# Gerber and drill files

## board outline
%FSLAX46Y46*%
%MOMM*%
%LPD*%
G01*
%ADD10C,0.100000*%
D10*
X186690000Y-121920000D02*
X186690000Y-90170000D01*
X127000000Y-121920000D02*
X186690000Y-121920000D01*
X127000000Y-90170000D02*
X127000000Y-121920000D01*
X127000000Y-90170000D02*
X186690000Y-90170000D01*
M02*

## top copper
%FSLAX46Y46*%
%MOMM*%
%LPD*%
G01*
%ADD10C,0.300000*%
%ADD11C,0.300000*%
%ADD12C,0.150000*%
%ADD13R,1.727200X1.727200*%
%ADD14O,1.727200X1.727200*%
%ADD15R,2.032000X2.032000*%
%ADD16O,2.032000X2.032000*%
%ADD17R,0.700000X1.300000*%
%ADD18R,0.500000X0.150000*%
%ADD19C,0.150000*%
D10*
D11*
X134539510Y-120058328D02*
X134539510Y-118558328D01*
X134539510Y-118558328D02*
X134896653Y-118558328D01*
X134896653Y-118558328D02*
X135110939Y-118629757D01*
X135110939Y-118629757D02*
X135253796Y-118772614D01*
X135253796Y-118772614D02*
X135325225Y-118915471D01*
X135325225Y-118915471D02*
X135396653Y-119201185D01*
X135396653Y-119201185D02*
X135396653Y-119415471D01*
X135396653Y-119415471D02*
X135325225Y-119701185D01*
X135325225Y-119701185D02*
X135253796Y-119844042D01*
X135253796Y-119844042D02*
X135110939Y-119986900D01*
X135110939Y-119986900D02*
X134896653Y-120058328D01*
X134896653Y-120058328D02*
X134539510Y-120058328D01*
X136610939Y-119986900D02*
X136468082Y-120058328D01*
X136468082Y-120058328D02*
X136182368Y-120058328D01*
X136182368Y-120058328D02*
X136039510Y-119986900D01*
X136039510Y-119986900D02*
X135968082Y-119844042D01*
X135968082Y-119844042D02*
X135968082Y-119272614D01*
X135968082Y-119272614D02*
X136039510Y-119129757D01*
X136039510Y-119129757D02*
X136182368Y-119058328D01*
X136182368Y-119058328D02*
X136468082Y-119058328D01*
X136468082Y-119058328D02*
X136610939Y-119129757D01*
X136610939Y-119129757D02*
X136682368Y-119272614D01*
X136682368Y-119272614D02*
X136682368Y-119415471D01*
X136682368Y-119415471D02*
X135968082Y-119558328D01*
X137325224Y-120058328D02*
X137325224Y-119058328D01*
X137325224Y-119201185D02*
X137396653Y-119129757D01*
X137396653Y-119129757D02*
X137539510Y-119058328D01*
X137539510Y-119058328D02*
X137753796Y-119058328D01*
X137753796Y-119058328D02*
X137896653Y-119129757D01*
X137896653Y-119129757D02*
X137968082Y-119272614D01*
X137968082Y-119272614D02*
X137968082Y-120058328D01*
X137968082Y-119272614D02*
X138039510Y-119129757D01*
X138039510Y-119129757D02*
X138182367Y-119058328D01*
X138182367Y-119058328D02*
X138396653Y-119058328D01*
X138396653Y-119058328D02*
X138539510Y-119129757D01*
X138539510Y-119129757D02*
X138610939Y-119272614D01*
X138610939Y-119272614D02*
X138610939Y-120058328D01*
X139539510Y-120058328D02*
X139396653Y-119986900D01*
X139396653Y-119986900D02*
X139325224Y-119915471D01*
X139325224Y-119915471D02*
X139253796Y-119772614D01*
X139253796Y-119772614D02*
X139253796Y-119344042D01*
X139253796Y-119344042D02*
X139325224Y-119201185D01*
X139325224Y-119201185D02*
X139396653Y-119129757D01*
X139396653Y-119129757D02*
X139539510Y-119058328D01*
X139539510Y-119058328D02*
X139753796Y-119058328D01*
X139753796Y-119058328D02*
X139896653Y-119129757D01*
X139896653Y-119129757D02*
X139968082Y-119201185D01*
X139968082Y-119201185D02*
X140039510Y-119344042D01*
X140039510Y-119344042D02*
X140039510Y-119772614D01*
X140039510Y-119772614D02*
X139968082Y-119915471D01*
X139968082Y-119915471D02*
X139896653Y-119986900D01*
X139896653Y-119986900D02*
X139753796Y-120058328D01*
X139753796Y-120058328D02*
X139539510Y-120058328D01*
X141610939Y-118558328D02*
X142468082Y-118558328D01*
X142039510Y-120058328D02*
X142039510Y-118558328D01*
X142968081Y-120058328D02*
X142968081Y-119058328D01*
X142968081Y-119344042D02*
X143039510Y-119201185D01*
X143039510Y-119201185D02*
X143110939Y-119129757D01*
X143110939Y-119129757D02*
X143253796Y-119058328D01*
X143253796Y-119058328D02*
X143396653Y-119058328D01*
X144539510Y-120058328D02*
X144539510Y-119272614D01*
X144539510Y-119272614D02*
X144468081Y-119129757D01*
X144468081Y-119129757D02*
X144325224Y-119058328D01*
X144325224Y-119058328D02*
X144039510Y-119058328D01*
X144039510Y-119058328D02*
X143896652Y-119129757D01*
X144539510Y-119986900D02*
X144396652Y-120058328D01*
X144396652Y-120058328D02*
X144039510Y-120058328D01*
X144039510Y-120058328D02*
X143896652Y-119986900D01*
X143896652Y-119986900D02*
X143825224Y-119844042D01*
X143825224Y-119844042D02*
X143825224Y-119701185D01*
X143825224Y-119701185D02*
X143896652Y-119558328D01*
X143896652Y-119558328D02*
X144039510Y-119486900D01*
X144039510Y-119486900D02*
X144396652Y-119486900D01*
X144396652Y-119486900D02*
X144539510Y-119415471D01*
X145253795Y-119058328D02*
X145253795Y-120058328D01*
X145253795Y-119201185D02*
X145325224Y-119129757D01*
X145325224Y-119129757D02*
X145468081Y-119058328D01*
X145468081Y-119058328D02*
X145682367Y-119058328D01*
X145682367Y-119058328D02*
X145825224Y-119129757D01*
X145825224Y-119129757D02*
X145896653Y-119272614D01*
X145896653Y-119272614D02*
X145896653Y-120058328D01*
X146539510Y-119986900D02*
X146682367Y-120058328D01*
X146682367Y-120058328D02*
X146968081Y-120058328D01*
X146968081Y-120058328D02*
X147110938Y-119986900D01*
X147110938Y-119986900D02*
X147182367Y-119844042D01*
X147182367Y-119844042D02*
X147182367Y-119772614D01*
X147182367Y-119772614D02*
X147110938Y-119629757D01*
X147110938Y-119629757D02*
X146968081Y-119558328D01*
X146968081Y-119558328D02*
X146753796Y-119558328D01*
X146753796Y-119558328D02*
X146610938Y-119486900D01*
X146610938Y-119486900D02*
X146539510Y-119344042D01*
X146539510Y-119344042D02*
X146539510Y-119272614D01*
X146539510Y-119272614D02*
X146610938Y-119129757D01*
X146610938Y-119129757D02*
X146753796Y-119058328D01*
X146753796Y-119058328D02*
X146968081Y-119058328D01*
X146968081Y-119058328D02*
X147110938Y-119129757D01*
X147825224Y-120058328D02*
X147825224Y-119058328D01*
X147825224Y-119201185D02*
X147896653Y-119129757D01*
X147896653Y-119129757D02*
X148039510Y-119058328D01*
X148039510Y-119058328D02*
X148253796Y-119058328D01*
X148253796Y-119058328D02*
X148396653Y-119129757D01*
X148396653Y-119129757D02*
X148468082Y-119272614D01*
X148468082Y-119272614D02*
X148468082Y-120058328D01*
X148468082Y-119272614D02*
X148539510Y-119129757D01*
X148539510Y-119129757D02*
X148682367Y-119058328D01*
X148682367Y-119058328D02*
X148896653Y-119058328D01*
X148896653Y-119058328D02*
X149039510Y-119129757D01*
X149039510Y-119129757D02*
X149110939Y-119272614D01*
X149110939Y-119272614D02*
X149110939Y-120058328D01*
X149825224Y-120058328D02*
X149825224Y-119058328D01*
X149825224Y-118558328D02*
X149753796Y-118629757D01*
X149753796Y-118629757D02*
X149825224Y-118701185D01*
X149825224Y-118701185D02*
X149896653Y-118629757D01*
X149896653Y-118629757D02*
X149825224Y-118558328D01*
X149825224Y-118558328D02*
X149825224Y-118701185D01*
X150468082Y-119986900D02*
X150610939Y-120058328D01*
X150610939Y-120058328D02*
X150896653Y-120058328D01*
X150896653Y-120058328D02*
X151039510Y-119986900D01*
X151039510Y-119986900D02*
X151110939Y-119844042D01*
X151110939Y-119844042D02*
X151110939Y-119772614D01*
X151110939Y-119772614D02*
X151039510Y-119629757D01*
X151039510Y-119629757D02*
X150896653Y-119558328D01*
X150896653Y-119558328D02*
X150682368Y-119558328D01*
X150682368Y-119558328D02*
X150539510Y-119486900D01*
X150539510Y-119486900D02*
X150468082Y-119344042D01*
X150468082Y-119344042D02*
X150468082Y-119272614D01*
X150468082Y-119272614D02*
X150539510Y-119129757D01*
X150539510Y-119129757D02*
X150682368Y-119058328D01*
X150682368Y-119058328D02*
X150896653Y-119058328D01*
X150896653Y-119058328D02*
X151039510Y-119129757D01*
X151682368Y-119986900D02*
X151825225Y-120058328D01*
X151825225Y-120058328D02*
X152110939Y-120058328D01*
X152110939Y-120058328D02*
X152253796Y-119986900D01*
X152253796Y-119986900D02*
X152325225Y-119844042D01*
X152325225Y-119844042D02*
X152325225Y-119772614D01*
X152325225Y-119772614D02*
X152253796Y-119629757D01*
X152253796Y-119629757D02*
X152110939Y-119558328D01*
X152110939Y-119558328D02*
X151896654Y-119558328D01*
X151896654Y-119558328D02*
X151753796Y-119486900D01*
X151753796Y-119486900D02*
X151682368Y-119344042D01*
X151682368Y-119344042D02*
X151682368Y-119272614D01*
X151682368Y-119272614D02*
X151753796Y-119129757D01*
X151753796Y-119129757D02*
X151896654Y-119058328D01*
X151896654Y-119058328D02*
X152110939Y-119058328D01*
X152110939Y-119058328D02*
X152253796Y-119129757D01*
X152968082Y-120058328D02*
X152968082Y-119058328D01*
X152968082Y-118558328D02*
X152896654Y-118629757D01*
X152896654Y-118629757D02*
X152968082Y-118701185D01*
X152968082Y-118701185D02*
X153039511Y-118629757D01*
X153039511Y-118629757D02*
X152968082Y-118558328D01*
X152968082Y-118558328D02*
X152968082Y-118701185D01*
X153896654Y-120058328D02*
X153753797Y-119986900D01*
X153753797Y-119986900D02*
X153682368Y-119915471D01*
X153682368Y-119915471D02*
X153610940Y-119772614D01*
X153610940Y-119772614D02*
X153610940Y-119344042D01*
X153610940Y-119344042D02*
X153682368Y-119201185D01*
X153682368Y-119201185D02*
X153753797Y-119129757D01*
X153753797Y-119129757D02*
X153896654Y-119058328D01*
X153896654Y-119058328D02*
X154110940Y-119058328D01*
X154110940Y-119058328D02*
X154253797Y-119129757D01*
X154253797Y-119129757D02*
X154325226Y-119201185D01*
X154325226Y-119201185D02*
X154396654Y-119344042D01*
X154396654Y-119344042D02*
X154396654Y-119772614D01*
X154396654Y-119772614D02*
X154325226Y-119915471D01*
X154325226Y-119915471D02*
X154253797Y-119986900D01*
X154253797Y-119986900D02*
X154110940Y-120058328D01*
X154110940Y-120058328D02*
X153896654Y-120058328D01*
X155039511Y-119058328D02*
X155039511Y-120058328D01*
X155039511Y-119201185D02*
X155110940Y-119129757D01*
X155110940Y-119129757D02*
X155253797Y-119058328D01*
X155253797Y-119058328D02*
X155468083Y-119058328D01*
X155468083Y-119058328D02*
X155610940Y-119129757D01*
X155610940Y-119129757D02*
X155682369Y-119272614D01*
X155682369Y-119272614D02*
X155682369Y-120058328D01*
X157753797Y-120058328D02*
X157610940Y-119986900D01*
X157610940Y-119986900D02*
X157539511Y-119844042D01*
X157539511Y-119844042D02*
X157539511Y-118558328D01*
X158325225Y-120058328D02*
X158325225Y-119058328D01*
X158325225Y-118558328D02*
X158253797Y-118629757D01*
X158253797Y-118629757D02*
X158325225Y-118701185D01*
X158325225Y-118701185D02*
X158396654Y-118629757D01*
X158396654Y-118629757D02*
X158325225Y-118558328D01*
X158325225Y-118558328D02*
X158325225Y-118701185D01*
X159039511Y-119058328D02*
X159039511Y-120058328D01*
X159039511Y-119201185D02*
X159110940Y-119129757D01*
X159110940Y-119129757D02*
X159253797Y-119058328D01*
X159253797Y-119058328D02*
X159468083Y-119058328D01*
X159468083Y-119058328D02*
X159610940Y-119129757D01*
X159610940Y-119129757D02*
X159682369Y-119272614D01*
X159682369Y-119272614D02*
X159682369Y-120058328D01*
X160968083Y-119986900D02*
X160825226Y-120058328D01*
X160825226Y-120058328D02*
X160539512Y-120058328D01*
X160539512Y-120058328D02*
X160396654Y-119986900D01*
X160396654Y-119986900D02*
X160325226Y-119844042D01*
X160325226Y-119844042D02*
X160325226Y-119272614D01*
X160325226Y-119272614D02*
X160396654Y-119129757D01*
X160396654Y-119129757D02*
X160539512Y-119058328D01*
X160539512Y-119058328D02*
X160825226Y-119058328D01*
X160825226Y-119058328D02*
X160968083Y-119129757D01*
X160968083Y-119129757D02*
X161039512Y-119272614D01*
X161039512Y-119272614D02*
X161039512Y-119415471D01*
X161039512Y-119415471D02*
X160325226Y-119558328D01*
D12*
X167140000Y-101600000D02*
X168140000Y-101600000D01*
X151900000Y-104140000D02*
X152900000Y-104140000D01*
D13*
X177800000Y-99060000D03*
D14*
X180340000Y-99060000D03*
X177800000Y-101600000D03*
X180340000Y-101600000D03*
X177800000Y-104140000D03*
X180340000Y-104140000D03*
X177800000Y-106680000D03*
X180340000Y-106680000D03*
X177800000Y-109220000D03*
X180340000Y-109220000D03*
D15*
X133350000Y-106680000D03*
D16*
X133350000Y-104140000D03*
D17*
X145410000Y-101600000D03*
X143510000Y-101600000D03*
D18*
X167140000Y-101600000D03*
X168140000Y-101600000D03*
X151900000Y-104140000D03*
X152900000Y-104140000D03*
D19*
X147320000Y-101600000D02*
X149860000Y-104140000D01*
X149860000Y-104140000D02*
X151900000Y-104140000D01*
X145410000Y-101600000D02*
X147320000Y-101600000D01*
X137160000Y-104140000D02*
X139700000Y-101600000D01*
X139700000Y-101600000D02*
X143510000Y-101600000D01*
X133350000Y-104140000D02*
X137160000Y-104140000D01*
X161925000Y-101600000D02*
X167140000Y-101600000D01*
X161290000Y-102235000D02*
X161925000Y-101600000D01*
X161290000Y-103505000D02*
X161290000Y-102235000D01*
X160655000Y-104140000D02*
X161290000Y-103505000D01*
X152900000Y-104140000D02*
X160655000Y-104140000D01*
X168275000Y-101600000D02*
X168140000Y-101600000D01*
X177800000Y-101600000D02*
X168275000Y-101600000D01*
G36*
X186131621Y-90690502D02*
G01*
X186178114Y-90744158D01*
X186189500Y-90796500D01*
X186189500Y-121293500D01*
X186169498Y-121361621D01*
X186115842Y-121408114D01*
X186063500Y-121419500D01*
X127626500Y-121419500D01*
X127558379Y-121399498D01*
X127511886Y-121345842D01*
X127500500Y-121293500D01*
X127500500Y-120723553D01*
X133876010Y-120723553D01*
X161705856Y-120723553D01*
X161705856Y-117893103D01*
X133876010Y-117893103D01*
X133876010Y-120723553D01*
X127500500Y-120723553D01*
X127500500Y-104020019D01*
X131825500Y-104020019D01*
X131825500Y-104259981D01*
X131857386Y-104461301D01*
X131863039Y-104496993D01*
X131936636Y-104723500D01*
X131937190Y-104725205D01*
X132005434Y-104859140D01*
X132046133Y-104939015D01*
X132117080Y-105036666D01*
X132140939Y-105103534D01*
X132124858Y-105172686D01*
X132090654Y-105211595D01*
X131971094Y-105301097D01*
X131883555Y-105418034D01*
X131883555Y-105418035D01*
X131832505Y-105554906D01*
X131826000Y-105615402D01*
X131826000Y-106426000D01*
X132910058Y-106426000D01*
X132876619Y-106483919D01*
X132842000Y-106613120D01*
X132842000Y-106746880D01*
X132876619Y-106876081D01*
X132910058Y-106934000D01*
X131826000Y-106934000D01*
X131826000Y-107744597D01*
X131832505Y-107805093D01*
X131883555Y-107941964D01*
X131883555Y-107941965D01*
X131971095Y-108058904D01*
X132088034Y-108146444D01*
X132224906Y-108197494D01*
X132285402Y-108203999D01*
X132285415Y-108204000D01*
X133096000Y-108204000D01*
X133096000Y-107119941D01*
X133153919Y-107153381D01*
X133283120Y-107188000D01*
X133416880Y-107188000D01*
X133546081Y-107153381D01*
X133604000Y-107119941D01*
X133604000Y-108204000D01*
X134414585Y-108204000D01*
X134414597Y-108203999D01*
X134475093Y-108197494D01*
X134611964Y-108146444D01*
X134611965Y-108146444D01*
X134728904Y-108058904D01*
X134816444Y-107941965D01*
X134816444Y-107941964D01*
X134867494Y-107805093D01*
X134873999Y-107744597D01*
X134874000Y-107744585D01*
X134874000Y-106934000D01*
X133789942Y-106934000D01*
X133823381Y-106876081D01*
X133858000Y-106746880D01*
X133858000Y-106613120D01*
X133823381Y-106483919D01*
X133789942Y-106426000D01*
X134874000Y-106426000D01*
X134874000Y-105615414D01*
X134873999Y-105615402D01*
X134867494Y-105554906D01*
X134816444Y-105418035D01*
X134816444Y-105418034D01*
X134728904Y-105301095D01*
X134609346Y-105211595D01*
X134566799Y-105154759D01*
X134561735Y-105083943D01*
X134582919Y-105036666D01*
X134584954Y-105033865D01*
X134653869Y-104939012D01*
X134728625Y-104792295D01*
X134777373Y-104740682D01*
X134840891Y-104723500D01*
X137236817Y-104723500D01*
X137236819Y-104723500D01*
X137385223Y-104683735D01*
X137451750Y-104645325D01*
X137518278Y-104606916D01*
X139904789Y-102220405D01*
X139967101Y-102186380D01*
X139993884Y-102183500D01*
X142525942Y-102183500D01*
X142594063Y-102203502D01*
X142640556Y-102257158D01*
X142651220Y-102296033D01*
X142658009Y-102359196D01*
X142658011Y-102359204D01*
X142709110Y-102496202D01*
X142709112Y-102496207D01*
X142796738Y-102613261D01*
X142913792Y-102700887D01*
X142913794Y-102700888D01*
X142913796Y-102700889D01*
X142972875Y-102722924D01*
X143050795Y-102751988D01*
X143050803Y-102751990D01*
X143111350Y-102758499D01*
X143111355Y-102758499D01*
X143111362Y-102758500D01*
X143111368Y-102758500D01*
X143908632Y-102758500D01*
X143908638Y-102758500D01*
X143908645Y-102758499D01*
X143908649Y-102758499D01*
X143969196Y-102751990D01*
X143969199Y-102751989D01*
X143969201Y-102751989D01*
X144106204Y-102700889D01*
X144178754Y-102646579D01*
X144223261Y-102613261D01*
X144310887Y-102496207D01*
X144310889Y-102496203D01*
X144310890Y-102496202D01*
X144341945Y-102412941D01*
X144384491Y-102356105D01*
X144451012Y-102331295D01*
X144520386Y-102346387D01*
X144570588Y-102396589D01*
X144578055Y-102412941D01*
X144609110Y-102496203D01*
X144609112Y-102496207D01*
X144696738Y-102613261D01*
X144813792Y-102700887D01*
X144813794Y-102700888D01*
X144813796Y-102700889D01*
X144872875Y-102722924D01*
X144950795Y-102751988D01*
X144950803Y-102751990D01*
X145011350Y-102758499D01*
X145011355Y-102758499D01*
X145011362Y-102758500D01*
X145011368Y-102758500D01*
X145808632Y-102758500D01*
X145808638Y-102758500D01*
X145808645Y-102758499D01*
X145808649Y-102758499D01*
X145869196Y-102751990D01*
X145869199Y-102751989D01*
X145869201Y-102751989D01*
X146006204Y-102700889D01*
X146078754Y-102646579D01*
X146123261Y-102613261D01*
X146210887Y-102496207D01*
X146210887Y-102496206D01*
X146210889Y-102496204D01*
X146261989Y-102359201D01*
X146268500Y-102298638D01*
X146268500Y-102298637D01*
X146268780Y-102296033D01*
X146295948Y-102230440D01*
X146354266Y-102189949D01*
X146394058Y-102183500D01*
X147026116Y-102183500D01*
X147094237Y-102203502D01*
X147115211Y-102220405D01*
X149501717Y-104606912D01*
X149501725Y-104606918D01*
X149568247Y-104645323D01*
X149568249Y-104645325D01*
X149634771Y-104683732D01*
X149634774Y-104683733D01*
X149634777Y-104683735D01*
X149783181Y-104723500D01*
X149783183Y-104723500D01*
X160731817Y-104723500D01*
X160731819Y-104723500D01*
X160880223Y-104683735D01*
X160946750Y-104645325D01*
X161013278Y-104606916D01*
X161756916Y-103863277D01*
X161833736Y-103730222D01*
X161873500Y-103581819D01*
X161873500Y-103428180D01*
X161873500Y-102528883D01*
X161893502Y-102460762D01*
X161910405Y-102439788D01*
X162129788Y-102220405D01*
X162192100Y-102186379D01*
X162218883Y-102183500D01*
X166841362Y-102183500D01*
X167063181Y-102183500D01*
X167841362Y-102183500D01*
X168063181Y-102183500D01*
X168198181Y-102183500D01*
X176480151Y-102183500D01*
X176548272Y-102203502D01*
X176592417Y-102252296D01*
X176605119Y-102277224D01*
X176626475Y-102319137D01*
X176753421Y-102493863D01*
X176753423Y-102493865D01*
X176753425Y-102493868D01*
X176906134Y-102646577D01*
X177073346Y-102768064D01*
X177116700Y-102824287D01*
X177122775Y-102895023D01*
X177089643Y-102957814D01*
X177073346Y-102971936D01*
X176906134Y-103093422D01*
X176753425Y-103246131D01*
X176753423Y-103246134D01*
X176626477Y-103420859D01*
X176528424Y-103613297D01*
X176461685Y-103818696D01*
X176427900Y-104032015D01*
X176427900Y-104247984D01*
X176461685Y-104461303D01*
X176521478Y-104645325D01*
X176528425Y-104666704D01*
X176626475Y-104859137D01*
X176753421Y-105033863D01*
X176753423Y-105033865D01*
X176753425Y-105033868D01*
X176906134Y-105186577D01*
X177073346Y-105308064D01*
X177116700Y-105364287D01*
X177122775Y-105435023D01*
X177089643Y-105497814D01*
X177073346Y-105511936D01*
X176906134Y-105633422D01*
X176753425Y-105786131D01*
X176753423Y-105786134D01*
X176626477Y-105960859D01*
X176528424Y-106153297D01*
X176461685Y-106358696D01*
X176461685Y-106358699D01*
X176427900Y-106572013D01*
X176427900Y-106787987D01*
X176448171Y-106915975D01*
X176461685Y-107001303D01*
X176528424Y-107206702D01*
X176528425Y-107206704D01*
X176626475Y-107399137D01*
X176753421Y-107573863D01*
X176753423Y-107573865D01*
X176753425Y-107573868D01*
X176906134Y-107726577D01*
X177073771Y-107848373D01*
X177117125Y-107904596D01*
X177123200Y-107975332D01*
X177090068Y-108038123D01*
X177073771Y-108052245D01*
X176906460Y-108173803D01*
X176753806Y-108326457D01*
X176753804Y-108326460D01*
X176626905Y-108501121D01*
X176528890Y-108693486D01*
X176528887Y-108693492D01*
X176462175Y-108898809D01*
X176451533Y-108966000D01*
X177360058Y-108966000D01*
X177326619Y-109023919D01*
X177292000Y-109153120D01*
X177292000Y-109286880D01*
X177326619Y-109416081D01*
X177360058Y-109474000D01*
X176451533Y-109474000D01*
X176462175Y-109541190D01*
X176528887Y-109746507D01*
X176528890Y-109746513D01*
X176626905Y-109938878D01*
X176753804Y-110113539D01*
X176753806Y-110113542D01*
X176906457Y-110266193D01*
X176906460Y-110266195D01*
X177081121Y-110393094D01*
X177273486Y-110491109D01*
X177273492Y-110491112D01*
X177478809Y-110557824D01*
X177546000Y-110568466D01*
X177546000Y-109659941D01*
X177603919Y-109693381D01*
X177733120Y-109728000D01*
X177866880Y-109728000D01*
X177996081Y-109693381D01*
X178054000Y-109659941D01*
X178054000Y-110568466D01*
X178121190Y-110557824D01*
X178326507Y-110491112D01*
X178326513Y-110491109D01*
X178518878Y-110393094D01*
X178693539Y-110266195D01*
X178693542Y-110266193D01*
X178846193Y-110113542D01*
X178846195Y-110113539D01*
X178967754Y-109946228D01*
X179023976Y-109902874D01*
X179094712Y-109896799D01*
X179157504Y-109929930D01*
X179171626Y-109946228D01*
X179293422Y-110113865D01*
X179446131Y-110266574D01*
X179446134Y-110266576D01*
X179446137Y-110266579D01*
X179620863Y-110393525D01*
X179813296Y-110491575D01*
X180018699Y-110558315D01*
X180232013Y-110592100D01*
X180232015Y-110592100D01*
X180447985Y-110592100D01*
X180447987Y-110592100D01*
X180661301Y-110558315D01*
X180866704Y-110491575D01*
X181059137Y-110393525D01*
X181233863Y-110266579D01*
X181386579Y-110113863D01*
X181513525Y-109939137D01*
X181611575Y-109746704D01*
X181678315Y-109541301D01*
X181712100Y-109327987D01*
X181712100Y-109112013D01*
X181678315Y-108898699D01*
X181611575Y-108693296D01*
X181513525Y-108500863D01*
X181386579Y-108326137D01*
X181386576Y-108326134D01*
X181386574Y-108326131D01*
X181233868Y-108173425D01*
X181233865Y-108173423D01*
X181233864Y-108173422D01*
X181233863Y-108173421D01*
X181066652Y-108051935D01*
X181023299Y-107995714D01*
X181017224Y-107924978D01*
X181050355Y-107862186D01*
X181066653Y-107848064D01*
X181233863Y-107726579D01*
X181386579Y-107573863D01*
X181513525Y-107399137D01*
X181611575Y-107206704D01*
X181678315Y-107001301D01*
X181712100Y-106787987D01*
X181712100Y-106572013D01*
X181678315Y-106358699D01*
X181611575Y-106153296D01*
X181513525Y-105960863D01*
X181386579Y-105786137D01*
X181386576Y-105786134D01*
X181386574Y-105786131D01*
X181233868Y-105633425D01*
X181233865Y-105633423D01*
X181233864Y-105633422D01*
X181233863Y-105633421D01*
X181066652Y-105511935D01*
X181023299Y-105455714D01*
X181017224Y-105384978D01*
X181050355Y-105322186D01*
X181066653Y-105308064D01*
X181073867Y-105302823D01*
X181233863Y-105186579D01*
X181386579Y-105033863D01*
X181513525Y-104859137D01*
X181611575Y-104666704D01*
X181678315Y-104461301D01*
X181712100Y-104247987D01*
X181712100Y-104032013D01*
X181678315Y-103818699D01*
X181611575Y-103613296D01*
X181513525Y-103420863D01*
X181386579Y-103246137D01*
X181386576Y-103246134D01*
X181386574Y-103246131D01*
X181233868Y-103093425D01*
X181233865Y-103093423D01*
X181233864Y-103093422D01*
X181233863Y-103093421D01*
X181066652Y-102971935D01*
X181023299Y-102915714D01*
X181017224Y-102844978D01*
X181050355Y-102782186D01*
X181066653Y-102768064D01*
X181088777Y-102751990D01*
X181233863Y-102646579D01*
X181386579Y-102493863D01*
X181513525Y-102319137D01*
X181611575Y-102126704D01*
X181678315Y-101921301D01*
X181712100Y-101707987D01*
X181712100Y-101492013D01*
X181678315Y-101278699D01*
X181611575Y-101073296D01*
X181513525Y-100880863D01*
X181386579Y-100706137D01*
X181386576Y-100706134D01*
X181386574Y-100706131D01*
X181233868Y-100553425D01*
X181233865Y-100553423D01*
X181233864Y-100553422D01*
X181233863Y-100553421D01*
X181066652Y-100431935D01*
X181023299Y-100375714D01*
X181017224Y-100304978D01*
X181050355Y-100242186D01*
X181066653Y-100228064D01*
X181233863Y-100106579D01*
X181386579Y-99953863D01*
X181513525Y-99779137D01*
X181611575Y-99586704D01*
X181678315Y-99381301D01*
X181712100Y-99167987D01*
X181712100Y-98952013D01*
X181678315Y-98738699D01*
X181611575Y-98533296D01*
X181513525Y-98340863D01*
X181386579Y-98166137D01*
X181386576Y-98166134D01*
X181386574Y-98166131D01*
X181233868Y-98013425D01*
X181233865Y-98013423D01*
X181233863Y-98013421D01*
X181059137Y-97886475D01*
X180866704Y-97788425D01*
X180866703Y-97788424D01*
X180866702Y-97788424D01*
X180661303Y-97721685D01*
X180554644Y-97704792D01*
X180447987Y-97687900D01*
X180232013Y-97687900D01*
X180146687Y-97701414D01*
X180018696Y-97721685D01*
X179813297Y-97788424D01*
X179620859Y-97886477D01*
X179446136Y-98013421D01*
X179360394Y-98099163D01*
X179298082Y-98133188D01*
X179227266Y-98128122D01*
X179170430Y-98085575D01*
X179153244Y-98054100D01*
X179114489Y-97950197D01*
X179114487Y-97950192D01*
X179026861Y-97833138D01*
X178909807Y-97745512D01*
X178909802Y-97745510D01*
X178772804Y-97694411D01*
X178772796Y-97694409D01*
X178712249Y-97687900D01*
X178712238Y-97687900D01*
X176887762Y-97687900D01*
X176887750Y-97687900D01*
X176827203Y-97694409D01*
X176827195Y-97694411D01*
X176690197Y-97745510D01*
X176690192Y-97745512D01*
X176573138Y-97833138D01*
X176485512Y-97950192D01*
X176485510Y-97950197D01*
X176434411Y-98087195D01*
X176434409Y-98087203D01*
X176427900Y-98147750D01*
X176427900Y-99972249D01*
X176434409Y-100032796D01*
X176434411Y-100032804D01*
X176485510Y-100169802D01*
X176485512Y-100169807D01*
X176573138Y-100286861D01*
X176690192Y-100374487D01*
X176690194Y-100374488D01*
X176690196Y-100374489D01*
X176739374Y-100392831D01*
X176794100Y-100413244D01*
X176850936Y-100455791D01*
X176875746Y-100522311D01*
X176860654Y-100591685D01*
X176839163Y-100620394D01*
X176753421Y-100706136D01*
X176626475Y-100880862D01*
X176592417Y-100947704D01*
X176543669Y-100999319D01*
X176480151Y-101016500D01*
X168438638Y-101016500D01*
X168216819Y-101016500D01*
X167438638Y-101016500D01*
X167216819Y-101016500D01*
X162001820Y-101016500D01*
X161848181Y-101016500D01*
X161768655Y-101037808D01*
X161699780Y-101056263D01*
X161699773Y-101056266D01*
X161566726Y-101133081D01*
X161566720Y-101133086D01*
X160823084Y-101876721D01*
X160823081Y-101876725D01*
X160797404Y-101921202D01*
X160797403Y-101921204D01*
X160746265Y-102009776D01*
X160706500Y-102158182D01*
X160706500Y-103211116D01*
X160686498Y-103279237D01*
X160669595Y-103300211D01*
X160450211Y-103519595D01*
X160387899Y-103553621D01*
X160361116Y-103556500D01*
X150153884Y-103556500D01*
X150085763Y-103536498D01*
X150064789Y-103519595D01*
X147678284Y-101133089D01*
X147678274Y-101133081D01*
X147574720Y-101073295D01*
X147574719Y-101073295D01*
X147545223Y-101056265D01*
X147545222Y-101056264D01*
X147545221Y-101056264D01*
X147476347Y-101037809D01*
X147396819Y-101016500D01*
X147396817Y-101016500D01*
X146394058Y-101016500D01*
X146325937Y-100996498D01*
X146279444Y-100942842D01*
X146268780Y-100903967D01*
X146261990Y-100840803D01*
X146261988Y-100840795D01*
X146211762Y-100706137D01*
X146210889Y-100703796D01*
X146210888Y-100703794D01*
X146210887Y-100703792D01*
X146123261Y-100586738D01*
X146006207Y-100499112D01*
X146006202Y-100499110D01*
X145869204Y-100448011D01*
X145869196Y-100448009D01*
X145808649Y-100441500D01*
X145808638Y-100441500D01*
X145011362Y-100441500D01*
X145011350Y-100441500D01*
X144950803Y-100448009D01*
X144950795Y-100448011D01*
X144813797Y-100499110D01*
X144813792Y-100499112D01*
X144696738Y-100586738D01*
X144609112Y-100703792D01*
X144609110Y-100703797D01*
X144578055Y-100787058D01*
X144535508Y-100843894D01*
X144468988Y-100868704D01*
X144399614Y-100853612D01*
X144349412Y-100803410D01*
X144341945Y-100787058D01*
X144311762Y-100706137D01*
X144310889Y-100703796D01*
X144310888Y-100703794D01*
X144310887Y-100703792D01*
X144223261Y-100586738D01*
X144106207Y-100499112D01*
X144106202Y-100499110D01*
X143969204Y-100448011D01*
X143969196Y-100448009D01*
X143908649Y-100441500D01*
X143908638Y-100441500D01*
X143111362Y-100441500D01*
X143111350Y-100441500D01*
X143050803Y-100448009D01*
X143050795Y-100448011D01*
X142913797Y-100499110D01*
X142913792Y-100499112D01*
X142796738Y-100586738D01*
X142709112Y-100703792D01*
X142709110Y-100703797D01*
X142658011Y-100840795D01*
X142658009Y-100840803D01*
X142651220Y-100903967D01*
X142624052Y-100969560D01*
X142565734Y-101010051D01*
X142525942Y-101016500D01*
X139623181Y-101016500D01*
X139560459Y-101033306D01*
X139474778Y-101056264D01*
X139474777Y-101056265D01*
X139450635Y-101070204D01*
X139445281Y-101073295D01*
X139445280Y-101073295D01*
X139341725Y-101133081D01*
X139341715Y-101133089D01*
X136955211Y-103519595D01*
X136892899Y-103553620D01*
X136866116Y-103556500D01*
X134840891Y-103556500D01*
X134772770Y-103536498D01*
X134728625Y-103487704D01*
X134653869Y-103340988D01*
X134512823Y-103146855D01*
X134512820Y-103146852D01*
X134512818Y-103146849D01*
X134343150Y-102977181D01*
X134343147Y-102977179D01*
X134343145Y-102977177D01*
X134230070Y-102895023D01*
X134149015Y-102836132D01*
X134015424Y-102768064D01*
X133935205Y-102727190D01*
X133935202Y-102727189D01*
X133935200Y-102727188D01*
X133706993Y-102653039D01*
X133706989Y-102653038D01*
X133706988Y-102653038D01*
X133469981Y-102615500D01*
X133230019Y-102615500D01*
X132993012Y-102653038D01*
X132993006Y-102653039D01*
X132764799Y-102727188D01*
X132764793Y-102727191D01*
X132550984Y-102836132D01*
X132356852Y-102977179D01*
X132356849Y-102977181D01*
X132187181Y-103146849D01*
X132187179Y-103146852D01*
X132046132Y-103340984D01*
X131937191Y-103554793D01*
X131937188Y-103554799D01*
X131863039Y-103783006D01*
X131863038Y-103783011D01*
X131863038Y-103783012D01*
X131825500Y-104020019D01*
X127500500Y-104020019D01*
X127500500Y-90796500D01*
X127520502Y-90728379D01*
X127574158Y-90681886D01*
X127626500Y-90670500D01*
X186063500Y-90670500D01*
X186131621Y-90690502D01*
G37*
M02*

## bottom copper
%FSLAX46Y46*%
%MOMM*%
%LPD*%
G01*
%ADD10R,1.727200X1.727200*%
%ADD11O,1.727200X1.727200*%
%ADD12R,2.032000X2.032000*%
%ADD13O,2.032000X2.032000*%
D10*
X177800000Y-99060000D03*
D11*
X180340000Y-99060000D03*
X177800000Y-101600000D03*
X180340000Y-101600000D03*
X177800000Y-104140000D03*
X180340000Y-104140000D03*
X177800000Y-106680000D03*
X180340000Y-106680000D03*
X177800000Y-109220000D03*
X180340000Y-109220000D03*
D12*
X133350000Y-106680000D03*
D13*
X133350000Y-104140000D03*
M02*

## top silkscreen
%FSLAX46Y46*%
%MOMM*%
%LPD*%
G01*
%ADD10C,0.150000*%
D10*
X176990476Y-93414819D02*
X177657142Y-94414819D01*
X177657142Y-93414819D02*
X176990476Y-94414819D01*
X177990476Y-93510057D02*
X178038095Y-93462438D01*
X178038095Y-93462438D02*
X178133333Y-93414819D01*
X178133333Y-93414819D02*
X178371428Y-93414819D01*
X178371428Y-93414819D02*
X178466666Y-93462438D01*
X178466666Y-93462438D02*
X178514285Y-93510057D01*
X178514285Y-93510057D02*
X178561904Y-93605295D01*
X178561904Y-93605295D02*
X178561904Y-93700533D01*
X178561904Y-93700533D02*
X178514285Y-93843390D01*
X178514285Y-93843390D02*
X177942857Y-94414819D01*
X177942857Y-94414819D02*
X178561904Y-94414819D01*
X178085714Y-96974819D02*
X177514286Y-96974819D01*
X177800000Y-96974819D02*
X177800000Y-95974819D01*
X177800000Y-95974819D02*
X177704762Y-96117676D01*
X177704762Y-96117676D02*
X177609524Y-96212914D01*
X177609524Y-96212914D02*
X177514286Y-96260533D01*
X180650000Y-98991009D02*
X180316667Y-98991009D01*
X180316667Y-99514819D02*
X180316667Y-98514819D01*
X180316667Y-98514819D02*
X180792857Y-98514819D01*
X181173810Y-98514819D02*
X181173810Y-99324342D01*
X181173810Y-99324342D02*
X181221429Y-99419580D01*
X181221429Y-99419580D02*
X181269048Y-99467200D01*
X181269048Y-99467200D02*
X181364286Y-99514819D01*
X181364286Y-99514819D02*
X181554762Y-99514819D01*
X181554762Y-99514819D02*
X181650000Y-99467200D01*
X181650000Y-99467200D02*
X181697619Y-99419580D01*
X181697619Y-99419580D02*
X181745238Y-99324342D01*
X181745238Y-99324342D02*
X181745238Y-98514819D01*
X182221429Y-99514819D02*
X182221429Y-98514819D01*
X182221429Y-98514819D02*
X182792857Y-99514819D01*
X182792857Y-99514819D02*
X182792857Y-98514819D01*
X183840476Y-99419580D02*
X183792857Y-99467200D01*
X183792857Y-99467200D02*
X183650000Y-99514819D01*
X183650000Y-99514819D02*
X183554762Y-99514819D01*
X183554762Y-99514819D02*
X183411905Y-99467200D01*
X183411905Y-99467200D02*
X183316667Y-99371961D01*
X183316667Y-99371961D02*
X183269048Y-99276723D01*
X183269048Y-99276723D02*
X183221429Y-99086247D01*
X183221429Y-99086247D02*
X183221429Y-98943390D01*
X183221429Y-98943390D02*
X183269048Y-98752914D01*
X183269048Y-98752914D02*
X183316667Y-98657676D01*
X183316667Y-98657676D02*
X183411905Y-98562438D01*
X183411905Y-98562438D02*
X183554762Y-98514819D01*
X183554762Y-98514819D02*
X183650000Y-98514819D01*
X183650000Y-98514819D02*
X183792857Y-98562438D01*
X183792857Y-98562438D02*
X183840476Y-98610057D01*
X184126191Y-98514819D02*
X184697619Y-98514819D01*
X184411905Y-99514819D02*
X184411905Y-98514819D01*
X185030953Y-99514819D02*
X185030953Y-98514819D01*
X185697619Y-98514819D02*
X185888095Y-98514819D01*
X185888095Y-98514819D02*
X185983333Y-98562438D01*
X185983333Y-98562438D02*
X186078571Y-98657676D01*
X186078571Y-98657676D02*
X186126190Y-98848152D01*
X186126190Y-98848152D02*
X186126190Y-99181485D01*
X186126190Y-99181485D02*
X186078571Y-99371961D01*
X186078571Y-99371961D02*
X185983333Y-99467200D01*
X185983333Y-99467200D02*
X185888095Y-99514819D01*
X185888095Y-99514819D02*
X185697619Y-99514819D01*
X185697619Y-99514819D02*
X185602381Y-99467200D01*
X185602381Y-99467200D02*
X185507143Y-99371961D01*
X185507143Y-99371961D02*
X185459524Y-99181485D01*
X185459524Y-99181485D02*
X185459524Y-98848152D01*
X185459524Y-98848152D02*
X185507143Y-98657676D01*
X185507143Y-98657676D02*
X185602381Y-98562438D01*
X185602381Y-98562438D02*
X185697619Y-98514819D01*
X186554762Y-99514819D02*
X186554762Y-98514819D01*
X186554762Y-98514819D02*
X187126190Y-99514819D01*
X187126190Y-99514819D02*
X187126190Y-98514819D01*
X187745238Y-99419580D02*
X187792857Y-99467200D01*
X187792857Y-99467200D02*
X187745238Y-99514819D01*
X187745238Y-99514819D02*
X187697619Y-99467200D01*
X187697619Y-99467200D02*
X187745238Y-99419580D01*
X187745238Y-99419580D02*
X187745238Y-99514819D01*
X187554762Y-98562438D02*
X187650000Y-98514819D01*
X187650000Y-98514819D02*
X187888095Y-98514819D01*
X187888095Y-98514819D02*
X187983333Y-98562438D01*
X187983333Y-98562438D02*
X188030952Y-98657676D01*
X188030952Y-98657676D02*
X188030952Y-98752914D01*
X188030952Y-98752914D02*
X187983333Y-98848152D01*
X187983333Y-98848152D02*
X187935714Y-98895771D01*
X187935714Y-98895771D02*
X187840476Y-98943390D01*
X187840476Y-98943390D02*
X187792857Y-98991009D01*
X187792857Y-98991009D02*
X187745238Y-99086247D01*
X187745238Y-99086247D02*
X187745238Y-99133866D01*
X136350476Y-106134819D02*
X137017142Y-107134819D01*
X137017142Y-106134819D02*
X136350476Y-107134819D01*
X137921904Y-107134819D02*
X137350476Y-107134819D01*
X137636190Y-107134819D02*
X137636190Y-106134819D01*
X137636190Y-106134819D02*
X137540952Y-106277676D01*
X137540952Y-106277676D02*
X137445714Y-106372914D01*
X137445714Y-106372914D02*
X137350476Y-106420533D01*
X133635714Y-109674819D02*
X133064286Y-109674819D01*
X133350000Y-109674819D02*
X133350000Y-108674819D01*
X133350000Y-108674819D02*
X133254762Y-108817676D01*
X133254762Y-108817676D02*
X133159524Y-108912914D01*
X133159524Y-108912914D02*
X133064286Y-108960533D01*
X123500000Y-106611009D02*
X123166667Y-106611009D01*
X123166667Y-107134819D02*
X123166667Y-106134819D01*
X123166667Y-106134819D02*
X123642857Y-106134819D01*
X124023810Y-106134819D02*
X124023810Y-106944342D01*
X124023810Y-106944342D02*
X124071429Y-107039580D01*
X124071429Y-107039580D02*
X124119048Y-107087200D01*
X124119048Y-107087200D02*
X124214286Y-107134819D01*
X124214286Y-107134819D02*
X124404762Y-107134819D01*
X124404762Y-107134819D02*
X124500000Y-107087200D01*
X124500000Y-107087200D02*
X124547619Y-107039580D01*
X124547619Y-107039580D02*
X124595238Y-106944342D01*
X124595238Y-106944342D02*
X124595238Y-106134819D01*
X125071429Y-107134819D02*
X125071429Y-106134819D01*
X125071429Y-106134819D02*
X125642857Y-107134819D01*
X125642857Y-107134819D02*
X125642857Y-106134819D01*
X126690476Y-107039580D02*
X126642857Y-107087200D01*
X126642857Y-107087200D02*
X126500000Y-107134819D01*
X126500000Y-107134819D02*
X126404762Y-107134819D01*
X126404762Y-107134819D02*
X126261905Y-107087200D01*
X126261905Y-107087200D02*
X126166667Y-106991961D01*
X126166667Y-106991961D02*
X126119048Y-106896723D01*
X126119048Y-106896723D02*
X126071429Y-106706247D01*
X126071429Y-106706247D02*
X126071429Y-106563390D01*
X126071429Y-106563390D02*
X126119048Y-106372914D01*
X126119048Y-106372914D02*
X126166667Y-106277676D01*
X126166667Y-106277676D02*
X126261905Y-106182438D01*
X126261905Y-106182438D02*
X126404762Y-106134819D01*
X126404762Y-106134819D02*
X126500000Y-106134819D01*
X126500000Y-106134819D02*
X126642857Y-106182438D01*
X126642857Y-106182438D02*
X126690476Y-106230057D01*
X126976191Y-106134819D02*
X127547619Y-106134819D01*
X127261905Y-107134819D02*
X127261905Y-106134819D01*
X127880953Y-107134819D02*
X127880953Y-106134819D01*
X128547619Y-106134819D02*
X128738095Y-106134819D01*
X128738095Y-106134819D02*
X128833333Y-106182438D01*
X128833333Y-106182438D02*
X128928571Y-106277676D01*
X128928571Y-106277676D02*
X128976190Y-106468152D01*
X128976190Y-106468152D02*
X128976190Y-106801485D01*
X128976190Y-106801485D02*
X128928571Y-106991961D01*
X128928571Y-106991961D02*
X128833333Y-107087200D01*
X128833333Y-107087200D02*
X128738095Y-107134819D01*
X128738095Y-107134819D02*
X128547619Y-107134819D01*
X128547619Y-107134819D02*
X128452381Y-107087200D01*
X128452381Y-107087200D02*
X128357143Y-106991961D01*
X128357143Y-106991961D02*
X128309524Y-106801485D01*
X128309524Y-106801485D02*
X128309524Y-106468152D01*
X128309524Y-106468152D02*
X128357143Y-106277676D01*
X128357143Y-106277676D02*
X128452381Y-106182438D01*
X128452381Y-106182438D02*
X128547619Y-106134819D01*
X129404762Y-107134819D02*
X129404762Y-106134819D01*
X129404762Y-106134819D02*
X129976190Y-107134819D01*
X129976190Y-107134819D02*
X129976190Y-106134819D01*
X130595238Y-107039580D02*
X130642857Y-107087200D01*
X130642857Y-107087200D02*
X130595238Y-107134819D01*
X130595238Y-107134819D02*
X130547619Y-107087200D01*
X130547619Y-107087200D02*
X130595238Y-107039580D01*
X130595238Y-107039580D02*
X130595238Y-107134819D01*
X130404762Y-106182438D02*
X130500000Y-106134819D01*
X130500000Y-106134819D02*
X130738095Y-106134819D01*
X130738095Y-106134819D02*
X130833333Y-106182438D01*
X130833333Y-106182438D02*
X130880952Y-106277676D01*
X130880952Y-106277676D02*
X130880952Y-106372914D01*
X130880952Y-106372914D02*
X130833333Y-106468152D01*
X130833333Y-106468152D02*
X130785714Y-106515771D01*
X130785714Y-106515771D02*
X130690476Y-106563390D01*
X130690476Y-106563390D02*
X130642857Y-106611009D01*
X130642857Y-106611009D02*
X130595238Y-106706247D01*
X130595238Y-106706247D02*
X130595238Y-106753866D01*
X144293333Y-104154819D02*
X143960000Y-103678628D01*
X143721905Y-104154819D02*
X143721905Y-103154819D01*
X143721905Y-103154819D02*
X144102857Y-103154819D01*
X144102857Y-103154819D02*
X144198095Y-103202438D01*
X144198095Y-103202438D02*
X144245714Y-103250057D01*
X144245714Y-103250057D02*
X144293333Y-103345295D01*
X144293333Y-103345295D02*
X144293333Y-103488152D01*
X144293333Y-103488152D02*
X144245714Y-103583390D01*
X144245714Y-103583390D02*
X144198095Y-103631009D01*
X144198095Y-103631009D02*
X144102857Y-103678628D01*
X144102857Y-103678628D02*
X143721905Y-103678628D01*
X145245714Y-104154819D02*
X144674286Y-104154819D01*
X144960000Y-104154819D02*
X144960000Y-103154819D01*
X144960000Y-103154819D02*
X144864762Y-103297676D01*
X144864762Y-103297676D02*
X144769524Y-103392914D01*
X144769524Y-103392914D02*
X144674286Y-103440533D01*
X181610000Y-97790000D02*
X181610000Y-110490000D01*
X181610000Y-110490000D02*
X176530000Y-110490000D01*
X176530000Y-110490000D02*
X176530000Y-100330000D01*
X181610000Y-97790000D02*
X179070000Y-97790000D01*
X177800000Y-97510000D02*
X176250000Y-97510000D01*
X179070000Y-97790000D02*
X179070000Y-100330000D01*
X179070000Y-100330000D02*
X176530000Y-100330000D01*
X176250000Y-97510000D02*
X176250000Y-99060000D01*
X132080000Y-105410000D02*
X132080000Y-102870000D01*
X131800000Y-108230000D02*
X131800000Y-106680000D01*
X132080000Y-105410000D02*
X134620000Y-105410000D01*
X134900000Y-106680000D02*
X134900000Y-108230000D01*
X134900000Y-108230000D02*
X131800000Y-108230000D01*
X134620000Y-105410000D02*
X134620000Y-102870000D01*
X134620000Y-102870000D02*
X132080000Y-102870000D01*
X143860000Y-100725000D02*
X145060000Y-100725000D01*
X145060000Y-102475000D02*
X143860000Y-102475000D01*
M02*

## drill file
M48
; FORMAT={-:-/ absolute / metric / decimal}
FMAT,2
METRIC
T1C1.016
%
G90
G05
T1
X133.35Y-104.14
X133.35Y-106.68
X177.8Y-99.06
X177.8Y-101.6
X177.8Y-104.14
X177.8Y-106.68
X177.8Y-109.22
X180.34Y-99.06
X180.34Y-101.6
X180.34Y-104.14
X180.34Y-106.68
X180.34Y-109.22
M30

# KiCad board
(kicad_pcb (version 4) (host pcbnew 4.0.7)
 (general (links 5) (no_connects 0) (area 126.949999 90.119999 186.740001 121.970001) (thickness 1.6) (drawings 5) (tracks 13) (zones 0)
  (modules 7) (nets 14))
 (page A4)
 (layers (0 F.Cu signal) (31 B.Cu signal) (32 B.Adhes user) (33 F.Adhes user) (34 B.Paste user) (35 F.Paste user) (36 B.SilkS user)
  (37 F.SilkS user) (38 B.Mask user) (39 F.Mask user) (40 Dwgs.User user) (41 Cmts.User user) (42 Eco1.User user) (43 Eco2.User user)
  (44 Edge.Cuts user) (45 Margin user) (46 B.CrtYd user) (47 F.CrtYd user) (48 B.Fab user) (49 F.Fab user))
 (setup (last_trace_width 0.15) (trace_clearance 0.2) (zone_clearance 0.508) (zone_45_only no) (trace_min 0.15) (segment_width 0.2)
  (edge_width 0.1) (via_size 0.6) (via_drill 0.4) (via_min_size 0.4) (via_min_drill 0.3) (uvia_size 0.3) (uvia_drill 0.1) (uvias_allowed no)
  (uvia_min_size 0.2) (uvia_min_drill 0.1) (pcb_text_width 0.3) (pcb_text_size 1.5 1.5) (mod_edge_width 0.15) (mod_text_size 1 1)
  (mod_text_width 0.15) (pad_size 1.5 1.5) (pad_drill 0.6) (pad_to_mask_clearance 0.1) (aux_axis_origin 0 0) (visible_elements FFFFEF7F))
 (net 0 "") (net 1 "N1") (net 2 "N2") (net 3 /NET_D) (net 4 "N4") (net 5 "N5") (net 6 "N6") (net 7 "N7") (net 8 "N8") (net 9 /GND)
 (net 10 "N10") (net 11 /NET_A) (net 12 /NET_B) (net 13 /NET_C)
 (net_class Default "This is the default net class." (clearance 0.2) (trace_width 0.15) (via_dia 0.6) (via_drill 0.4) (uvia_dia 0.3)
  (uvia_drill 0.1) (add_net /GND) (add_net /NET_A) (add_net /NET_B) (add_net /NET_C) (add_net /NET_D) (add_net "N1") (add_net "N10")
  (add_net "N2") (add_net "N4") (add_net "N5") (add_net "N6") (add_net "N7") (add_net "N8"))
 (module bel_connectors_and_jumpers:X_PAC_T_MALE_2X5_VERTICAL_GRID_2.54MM (layer F.Cu) (at 177.8 99.06)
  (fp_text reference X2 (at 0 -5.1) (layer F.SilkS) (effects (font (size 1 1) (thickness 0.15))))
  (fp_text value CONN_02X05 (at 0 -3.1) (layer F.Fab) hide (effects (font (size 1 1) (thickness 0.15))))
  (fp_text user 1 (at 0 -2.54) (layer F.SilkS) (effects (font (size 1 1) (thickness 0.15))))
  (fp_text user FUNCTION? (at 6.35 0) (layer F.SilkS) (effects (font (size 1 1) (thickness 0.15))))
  (fp_line (start 3.81 -1.27) (end 3.81 11.43) (layer F.SilkS) (width 0.15))
  (fp_line (start 3.81 11.43) (end -1.27 11.43) (layer F.SilkS) (width 0.15))
  (fp_line (start -1.27 11.43) (end -1.27 1.27) (layer F.SilkS) (width 0.15))
  (fp_line (start 3.81 -1.27) (end 1.27 -1.27) (layer F.SilkS) (width 0.15))
  (fp_line (start 0 -1.55) (end -1.55 -1.55) (layer F.SilkS) (width 0.15))
  (fp_line (start 1.27 -1.27) (end 1.27 1.27) (layer F.SilkS) (width 0.15))
  (fp_line (start 1.27 1.27) (end -1.27 1.27) (layer F.SilkS) (width 0.15))
  (fp_line (start -1.55 -1.55) (end -1.55 0) (layer F.SilkS) (width 0.15))
  (pad 1 thru_hole rect (at 0 0) (size 1.7272 1.7272) (drill 1.016) (layers *.Cu *.Mask) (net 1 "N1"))
  (pad 2 thru_hole oval (at 2.54 0) (size 1.7272 1.7272) (drill 1.016) (layers *.Cu *.Mask) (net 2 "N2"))
  (pad 3 thru_hole oval (at 0 2.54) (size 1.7272 1.7272) (drill 1.016) (layers *.Cu *.Mask) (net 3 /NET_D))
  (pad 4 thru_hole oval (at 2.54 2.54) (size 1.7272 1.7272) (drill 1.016) (layers *.Cu *.Mask) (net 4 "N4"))
  (pad 5 thru_hole oval (at 0 5.08) (size 1.7272 1.7272) (drill 1.016) (layers *.Cu *.Mask) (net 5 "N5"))
  (pad 6 thru_hole oval (at 2.54 5.08) (size 1.7272 1.7272) (drill 1.016) (layers *.Cu *.Mask) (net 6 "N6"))
  (pad 7 thru_hole oval (at 0 7.62) (size 1.7272 1.7272) (drill 1.016) (layers *.Cu *.Mask) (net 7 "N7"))
  (pad 8 thru_hole oval (at 2.54 7.62) (size 1.7272 1.7272) (drill 1.016) (layers *.Cu *.Mask) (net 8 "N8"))
  (pad 9 thru_hole oval (at 0 10.16) (size 1.7272 1.7272) (drill 1.016) (layers *.Cu *.Mask) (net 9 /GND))
  (pad 10 thru_hole oval (at 2.54 10.16) (size 1.7272 1.7272) (drill 1.016) (layers *.Cu *.Mask) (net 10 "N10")))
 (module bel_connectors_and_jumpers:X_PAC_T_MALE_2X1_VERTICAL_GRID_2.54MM (layer F.Cu) (at 133.35 106.68 180)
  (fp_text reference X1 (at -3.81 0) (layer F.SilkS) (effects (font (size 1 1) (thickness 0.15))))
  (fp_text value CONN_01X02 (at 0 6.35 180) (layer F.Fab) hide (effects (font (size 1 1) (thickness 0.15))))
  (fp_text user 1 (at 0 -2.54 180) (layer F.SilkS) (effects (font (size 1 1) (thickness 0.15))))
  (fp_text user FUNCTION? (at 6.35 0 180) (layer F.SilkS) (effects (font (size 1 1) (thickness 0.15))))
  (fp_line (start 1.27 1.27) (end 1.27 3.81) (layer F.SilkS) (width 0.15))
  (fp_line (start 1.55 -1.55) (end 1.55 0) (layer F.SilkS) (width 0.15))
  (fp_line (start 1.27 1.27) (end -1.27 1.27) (layer F.SilkS) (width 0.15))
  (fp_line (start -1.55 0) (end -1.55 -1.55) (layer F.SilkS) (width 0.15))
  (fp_line (start -1.55 -1.55) (end 1.55 -1.55) (layer F.SilkS) (width 0.15))
  (fp_line (start -1.27 1.27) (end -1.27 3.81) (layer F.SilkS) (width 0.15))
  (fp_line (start -1.27 3.81) (end 1.27 3.81) (layer F.SilkS) (width 0.15))
  (pad 1 thru_hole rect (at 0 0 180) (size 2.032 2.032) (drill 1.016) (layers *.Cu *.Mask) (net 9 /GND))
  (pad 2 thru_hole oval (at 0 2.54 180) (size 2.032 2.032) (drill 1.016) (layers *.Cu *.Mask) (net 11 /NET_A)))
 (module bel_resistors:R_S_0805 (layer F.Cu) (at 144.46 101.6 180)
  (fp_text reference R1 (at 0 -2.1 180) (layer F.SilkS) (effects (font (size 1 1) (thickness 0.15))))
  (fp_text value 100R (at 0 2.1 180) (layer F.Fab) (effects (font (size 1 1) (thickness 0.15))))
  (fp_line (start 0.6 0.875) (end -0.6 0.875) (layer F.SilkS) (width 0.15))
  (fp_line (start -0.6 -0.875) (end 0.6 -0.875) (layer F.SilkS) (width 0.15))
  (pad 1 smd rect (at -0.95 0 180) (size 0.7 1.3) (layers F.Cu F.Paste F.Mask) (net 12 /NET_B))
  (pad 2 smd rect (at 0.95 0 180) (size 0.7 1.3) (layers F.Cu F.Paste F.Mask) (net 11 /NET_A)))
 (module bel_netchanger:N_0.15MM (layer F.Cu) (at 167.64 101.6)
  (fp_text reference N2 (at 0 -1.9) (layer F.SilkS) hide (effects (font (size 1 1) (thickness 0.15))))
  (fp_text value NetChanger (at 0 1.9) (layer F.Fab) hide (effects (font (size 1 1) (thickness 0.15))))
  (fp_line (start -0.5 0) (end 0.5 0) (layer F.Cu) (width 0.15))
  (pad 1 smd rect (at -0.5 0) (size 0.5 0.15) (layers F.Cu) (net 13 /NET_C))
  (pad 2 smd rect (at 0.5 0) (size 0.5 0.15) (layers F.Cu) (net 3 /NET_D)))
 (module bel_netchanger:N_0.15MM (layer F.Cu) (at 152.4 104.14)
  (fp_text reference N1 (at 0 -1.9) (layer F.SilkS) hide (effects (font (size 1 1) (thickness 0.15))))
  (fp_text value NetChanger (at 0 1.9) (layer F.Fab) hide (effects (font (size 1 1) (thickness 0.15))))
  (fp_line (start -0.5 0) (end 0.5 0) (layer F.Cu) (width 0.15))
  (pad 1 smd rect (at -0.5 0) (size 0.5 0.15) (layers F.Cu) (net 12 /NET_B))
  (pad 2 smd rect (at 0.5 0) (size 0.5 0.15) (layers F.Cu) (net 13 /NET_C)))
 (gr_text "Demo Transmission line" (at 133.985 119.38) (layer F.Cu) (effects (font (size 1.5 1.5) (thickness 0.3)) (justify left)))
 (gr_line (start 186.69 121.92) (end 186.69 90.17) (angle 90) (layer Edge.Cuts) (width 0.1))
 (gr_line (start 127 121.92) (end 186.69 121.92) (angle 90) (layer Edge.Cuts) (width 0.1))
 (gr_line (start 127 90.17) (end 127 121.92) (angle 90) (layer Edge.Cuts) (width 0.1))
 (gr_line (start 127 90.17) (end 186.69 90.17) (angle 90) (layer Edge.Cuts) (width 0.1))
 (segment (start 147.32 101.6) (end 149.86 104.14) (width 0.15) (layer F.Cu) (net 12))
 (segment (start 149.86 104.14) (end 151.9 104.14) (width 0.15) (layer F.Cu) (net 12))
 (segment (start 145.41 101.6) (end 147.32 101.6) (width 0.15) (layer F.Cu) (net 12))
 (segment (start 137.16 104.14) (end 139.7 101.6) (width 0.15) (layer F.Cu) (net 11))
 (segment (start 139.7 101.6) (end 143.51 101.6) (width 0.15) (layer F.Cu) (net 11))
 (segment (start 133.35 104.14) (end 137.16 104.14) (width 0.15) (layer F.Cu) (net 11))
 (segment (start 161.925 101.6) (end 167.14 101.6) (width 0.15) (layer F.Cu) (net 13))
 (segment (start 161.29 102.235) (end 161.925 101.6) (width 0.15) (layer F.Cu) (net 13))
 (segment (start 161.29 103.505) (end 161.29 102.235) (width 0.15) (layer F.Cu) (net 13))
 (segment (start 160.655 104.14) (end 161.29 103.505) (width 0.15) (layer F.Cu) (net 13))
 (segment (start 152.9 104.14) (end 160.655 104.14) (width 0.15) (layer F.Cu) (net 13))
 (segment (start 168.275 101.6) (end 168.14 101.6) (width 0.15) (layer F.Cu) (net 3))
 (segment (start 177.8 101.6) (end 168.275 101.6) (width 0.15) (layer F.Cu) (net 3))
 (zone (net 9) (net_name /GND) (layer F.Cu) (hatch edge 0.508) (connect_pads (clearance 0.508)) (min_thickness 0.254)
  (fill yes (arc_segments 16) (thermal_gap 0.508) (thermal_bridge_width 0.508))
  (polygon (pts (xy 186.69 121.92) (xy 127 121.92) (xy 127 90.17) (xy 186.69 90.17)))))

